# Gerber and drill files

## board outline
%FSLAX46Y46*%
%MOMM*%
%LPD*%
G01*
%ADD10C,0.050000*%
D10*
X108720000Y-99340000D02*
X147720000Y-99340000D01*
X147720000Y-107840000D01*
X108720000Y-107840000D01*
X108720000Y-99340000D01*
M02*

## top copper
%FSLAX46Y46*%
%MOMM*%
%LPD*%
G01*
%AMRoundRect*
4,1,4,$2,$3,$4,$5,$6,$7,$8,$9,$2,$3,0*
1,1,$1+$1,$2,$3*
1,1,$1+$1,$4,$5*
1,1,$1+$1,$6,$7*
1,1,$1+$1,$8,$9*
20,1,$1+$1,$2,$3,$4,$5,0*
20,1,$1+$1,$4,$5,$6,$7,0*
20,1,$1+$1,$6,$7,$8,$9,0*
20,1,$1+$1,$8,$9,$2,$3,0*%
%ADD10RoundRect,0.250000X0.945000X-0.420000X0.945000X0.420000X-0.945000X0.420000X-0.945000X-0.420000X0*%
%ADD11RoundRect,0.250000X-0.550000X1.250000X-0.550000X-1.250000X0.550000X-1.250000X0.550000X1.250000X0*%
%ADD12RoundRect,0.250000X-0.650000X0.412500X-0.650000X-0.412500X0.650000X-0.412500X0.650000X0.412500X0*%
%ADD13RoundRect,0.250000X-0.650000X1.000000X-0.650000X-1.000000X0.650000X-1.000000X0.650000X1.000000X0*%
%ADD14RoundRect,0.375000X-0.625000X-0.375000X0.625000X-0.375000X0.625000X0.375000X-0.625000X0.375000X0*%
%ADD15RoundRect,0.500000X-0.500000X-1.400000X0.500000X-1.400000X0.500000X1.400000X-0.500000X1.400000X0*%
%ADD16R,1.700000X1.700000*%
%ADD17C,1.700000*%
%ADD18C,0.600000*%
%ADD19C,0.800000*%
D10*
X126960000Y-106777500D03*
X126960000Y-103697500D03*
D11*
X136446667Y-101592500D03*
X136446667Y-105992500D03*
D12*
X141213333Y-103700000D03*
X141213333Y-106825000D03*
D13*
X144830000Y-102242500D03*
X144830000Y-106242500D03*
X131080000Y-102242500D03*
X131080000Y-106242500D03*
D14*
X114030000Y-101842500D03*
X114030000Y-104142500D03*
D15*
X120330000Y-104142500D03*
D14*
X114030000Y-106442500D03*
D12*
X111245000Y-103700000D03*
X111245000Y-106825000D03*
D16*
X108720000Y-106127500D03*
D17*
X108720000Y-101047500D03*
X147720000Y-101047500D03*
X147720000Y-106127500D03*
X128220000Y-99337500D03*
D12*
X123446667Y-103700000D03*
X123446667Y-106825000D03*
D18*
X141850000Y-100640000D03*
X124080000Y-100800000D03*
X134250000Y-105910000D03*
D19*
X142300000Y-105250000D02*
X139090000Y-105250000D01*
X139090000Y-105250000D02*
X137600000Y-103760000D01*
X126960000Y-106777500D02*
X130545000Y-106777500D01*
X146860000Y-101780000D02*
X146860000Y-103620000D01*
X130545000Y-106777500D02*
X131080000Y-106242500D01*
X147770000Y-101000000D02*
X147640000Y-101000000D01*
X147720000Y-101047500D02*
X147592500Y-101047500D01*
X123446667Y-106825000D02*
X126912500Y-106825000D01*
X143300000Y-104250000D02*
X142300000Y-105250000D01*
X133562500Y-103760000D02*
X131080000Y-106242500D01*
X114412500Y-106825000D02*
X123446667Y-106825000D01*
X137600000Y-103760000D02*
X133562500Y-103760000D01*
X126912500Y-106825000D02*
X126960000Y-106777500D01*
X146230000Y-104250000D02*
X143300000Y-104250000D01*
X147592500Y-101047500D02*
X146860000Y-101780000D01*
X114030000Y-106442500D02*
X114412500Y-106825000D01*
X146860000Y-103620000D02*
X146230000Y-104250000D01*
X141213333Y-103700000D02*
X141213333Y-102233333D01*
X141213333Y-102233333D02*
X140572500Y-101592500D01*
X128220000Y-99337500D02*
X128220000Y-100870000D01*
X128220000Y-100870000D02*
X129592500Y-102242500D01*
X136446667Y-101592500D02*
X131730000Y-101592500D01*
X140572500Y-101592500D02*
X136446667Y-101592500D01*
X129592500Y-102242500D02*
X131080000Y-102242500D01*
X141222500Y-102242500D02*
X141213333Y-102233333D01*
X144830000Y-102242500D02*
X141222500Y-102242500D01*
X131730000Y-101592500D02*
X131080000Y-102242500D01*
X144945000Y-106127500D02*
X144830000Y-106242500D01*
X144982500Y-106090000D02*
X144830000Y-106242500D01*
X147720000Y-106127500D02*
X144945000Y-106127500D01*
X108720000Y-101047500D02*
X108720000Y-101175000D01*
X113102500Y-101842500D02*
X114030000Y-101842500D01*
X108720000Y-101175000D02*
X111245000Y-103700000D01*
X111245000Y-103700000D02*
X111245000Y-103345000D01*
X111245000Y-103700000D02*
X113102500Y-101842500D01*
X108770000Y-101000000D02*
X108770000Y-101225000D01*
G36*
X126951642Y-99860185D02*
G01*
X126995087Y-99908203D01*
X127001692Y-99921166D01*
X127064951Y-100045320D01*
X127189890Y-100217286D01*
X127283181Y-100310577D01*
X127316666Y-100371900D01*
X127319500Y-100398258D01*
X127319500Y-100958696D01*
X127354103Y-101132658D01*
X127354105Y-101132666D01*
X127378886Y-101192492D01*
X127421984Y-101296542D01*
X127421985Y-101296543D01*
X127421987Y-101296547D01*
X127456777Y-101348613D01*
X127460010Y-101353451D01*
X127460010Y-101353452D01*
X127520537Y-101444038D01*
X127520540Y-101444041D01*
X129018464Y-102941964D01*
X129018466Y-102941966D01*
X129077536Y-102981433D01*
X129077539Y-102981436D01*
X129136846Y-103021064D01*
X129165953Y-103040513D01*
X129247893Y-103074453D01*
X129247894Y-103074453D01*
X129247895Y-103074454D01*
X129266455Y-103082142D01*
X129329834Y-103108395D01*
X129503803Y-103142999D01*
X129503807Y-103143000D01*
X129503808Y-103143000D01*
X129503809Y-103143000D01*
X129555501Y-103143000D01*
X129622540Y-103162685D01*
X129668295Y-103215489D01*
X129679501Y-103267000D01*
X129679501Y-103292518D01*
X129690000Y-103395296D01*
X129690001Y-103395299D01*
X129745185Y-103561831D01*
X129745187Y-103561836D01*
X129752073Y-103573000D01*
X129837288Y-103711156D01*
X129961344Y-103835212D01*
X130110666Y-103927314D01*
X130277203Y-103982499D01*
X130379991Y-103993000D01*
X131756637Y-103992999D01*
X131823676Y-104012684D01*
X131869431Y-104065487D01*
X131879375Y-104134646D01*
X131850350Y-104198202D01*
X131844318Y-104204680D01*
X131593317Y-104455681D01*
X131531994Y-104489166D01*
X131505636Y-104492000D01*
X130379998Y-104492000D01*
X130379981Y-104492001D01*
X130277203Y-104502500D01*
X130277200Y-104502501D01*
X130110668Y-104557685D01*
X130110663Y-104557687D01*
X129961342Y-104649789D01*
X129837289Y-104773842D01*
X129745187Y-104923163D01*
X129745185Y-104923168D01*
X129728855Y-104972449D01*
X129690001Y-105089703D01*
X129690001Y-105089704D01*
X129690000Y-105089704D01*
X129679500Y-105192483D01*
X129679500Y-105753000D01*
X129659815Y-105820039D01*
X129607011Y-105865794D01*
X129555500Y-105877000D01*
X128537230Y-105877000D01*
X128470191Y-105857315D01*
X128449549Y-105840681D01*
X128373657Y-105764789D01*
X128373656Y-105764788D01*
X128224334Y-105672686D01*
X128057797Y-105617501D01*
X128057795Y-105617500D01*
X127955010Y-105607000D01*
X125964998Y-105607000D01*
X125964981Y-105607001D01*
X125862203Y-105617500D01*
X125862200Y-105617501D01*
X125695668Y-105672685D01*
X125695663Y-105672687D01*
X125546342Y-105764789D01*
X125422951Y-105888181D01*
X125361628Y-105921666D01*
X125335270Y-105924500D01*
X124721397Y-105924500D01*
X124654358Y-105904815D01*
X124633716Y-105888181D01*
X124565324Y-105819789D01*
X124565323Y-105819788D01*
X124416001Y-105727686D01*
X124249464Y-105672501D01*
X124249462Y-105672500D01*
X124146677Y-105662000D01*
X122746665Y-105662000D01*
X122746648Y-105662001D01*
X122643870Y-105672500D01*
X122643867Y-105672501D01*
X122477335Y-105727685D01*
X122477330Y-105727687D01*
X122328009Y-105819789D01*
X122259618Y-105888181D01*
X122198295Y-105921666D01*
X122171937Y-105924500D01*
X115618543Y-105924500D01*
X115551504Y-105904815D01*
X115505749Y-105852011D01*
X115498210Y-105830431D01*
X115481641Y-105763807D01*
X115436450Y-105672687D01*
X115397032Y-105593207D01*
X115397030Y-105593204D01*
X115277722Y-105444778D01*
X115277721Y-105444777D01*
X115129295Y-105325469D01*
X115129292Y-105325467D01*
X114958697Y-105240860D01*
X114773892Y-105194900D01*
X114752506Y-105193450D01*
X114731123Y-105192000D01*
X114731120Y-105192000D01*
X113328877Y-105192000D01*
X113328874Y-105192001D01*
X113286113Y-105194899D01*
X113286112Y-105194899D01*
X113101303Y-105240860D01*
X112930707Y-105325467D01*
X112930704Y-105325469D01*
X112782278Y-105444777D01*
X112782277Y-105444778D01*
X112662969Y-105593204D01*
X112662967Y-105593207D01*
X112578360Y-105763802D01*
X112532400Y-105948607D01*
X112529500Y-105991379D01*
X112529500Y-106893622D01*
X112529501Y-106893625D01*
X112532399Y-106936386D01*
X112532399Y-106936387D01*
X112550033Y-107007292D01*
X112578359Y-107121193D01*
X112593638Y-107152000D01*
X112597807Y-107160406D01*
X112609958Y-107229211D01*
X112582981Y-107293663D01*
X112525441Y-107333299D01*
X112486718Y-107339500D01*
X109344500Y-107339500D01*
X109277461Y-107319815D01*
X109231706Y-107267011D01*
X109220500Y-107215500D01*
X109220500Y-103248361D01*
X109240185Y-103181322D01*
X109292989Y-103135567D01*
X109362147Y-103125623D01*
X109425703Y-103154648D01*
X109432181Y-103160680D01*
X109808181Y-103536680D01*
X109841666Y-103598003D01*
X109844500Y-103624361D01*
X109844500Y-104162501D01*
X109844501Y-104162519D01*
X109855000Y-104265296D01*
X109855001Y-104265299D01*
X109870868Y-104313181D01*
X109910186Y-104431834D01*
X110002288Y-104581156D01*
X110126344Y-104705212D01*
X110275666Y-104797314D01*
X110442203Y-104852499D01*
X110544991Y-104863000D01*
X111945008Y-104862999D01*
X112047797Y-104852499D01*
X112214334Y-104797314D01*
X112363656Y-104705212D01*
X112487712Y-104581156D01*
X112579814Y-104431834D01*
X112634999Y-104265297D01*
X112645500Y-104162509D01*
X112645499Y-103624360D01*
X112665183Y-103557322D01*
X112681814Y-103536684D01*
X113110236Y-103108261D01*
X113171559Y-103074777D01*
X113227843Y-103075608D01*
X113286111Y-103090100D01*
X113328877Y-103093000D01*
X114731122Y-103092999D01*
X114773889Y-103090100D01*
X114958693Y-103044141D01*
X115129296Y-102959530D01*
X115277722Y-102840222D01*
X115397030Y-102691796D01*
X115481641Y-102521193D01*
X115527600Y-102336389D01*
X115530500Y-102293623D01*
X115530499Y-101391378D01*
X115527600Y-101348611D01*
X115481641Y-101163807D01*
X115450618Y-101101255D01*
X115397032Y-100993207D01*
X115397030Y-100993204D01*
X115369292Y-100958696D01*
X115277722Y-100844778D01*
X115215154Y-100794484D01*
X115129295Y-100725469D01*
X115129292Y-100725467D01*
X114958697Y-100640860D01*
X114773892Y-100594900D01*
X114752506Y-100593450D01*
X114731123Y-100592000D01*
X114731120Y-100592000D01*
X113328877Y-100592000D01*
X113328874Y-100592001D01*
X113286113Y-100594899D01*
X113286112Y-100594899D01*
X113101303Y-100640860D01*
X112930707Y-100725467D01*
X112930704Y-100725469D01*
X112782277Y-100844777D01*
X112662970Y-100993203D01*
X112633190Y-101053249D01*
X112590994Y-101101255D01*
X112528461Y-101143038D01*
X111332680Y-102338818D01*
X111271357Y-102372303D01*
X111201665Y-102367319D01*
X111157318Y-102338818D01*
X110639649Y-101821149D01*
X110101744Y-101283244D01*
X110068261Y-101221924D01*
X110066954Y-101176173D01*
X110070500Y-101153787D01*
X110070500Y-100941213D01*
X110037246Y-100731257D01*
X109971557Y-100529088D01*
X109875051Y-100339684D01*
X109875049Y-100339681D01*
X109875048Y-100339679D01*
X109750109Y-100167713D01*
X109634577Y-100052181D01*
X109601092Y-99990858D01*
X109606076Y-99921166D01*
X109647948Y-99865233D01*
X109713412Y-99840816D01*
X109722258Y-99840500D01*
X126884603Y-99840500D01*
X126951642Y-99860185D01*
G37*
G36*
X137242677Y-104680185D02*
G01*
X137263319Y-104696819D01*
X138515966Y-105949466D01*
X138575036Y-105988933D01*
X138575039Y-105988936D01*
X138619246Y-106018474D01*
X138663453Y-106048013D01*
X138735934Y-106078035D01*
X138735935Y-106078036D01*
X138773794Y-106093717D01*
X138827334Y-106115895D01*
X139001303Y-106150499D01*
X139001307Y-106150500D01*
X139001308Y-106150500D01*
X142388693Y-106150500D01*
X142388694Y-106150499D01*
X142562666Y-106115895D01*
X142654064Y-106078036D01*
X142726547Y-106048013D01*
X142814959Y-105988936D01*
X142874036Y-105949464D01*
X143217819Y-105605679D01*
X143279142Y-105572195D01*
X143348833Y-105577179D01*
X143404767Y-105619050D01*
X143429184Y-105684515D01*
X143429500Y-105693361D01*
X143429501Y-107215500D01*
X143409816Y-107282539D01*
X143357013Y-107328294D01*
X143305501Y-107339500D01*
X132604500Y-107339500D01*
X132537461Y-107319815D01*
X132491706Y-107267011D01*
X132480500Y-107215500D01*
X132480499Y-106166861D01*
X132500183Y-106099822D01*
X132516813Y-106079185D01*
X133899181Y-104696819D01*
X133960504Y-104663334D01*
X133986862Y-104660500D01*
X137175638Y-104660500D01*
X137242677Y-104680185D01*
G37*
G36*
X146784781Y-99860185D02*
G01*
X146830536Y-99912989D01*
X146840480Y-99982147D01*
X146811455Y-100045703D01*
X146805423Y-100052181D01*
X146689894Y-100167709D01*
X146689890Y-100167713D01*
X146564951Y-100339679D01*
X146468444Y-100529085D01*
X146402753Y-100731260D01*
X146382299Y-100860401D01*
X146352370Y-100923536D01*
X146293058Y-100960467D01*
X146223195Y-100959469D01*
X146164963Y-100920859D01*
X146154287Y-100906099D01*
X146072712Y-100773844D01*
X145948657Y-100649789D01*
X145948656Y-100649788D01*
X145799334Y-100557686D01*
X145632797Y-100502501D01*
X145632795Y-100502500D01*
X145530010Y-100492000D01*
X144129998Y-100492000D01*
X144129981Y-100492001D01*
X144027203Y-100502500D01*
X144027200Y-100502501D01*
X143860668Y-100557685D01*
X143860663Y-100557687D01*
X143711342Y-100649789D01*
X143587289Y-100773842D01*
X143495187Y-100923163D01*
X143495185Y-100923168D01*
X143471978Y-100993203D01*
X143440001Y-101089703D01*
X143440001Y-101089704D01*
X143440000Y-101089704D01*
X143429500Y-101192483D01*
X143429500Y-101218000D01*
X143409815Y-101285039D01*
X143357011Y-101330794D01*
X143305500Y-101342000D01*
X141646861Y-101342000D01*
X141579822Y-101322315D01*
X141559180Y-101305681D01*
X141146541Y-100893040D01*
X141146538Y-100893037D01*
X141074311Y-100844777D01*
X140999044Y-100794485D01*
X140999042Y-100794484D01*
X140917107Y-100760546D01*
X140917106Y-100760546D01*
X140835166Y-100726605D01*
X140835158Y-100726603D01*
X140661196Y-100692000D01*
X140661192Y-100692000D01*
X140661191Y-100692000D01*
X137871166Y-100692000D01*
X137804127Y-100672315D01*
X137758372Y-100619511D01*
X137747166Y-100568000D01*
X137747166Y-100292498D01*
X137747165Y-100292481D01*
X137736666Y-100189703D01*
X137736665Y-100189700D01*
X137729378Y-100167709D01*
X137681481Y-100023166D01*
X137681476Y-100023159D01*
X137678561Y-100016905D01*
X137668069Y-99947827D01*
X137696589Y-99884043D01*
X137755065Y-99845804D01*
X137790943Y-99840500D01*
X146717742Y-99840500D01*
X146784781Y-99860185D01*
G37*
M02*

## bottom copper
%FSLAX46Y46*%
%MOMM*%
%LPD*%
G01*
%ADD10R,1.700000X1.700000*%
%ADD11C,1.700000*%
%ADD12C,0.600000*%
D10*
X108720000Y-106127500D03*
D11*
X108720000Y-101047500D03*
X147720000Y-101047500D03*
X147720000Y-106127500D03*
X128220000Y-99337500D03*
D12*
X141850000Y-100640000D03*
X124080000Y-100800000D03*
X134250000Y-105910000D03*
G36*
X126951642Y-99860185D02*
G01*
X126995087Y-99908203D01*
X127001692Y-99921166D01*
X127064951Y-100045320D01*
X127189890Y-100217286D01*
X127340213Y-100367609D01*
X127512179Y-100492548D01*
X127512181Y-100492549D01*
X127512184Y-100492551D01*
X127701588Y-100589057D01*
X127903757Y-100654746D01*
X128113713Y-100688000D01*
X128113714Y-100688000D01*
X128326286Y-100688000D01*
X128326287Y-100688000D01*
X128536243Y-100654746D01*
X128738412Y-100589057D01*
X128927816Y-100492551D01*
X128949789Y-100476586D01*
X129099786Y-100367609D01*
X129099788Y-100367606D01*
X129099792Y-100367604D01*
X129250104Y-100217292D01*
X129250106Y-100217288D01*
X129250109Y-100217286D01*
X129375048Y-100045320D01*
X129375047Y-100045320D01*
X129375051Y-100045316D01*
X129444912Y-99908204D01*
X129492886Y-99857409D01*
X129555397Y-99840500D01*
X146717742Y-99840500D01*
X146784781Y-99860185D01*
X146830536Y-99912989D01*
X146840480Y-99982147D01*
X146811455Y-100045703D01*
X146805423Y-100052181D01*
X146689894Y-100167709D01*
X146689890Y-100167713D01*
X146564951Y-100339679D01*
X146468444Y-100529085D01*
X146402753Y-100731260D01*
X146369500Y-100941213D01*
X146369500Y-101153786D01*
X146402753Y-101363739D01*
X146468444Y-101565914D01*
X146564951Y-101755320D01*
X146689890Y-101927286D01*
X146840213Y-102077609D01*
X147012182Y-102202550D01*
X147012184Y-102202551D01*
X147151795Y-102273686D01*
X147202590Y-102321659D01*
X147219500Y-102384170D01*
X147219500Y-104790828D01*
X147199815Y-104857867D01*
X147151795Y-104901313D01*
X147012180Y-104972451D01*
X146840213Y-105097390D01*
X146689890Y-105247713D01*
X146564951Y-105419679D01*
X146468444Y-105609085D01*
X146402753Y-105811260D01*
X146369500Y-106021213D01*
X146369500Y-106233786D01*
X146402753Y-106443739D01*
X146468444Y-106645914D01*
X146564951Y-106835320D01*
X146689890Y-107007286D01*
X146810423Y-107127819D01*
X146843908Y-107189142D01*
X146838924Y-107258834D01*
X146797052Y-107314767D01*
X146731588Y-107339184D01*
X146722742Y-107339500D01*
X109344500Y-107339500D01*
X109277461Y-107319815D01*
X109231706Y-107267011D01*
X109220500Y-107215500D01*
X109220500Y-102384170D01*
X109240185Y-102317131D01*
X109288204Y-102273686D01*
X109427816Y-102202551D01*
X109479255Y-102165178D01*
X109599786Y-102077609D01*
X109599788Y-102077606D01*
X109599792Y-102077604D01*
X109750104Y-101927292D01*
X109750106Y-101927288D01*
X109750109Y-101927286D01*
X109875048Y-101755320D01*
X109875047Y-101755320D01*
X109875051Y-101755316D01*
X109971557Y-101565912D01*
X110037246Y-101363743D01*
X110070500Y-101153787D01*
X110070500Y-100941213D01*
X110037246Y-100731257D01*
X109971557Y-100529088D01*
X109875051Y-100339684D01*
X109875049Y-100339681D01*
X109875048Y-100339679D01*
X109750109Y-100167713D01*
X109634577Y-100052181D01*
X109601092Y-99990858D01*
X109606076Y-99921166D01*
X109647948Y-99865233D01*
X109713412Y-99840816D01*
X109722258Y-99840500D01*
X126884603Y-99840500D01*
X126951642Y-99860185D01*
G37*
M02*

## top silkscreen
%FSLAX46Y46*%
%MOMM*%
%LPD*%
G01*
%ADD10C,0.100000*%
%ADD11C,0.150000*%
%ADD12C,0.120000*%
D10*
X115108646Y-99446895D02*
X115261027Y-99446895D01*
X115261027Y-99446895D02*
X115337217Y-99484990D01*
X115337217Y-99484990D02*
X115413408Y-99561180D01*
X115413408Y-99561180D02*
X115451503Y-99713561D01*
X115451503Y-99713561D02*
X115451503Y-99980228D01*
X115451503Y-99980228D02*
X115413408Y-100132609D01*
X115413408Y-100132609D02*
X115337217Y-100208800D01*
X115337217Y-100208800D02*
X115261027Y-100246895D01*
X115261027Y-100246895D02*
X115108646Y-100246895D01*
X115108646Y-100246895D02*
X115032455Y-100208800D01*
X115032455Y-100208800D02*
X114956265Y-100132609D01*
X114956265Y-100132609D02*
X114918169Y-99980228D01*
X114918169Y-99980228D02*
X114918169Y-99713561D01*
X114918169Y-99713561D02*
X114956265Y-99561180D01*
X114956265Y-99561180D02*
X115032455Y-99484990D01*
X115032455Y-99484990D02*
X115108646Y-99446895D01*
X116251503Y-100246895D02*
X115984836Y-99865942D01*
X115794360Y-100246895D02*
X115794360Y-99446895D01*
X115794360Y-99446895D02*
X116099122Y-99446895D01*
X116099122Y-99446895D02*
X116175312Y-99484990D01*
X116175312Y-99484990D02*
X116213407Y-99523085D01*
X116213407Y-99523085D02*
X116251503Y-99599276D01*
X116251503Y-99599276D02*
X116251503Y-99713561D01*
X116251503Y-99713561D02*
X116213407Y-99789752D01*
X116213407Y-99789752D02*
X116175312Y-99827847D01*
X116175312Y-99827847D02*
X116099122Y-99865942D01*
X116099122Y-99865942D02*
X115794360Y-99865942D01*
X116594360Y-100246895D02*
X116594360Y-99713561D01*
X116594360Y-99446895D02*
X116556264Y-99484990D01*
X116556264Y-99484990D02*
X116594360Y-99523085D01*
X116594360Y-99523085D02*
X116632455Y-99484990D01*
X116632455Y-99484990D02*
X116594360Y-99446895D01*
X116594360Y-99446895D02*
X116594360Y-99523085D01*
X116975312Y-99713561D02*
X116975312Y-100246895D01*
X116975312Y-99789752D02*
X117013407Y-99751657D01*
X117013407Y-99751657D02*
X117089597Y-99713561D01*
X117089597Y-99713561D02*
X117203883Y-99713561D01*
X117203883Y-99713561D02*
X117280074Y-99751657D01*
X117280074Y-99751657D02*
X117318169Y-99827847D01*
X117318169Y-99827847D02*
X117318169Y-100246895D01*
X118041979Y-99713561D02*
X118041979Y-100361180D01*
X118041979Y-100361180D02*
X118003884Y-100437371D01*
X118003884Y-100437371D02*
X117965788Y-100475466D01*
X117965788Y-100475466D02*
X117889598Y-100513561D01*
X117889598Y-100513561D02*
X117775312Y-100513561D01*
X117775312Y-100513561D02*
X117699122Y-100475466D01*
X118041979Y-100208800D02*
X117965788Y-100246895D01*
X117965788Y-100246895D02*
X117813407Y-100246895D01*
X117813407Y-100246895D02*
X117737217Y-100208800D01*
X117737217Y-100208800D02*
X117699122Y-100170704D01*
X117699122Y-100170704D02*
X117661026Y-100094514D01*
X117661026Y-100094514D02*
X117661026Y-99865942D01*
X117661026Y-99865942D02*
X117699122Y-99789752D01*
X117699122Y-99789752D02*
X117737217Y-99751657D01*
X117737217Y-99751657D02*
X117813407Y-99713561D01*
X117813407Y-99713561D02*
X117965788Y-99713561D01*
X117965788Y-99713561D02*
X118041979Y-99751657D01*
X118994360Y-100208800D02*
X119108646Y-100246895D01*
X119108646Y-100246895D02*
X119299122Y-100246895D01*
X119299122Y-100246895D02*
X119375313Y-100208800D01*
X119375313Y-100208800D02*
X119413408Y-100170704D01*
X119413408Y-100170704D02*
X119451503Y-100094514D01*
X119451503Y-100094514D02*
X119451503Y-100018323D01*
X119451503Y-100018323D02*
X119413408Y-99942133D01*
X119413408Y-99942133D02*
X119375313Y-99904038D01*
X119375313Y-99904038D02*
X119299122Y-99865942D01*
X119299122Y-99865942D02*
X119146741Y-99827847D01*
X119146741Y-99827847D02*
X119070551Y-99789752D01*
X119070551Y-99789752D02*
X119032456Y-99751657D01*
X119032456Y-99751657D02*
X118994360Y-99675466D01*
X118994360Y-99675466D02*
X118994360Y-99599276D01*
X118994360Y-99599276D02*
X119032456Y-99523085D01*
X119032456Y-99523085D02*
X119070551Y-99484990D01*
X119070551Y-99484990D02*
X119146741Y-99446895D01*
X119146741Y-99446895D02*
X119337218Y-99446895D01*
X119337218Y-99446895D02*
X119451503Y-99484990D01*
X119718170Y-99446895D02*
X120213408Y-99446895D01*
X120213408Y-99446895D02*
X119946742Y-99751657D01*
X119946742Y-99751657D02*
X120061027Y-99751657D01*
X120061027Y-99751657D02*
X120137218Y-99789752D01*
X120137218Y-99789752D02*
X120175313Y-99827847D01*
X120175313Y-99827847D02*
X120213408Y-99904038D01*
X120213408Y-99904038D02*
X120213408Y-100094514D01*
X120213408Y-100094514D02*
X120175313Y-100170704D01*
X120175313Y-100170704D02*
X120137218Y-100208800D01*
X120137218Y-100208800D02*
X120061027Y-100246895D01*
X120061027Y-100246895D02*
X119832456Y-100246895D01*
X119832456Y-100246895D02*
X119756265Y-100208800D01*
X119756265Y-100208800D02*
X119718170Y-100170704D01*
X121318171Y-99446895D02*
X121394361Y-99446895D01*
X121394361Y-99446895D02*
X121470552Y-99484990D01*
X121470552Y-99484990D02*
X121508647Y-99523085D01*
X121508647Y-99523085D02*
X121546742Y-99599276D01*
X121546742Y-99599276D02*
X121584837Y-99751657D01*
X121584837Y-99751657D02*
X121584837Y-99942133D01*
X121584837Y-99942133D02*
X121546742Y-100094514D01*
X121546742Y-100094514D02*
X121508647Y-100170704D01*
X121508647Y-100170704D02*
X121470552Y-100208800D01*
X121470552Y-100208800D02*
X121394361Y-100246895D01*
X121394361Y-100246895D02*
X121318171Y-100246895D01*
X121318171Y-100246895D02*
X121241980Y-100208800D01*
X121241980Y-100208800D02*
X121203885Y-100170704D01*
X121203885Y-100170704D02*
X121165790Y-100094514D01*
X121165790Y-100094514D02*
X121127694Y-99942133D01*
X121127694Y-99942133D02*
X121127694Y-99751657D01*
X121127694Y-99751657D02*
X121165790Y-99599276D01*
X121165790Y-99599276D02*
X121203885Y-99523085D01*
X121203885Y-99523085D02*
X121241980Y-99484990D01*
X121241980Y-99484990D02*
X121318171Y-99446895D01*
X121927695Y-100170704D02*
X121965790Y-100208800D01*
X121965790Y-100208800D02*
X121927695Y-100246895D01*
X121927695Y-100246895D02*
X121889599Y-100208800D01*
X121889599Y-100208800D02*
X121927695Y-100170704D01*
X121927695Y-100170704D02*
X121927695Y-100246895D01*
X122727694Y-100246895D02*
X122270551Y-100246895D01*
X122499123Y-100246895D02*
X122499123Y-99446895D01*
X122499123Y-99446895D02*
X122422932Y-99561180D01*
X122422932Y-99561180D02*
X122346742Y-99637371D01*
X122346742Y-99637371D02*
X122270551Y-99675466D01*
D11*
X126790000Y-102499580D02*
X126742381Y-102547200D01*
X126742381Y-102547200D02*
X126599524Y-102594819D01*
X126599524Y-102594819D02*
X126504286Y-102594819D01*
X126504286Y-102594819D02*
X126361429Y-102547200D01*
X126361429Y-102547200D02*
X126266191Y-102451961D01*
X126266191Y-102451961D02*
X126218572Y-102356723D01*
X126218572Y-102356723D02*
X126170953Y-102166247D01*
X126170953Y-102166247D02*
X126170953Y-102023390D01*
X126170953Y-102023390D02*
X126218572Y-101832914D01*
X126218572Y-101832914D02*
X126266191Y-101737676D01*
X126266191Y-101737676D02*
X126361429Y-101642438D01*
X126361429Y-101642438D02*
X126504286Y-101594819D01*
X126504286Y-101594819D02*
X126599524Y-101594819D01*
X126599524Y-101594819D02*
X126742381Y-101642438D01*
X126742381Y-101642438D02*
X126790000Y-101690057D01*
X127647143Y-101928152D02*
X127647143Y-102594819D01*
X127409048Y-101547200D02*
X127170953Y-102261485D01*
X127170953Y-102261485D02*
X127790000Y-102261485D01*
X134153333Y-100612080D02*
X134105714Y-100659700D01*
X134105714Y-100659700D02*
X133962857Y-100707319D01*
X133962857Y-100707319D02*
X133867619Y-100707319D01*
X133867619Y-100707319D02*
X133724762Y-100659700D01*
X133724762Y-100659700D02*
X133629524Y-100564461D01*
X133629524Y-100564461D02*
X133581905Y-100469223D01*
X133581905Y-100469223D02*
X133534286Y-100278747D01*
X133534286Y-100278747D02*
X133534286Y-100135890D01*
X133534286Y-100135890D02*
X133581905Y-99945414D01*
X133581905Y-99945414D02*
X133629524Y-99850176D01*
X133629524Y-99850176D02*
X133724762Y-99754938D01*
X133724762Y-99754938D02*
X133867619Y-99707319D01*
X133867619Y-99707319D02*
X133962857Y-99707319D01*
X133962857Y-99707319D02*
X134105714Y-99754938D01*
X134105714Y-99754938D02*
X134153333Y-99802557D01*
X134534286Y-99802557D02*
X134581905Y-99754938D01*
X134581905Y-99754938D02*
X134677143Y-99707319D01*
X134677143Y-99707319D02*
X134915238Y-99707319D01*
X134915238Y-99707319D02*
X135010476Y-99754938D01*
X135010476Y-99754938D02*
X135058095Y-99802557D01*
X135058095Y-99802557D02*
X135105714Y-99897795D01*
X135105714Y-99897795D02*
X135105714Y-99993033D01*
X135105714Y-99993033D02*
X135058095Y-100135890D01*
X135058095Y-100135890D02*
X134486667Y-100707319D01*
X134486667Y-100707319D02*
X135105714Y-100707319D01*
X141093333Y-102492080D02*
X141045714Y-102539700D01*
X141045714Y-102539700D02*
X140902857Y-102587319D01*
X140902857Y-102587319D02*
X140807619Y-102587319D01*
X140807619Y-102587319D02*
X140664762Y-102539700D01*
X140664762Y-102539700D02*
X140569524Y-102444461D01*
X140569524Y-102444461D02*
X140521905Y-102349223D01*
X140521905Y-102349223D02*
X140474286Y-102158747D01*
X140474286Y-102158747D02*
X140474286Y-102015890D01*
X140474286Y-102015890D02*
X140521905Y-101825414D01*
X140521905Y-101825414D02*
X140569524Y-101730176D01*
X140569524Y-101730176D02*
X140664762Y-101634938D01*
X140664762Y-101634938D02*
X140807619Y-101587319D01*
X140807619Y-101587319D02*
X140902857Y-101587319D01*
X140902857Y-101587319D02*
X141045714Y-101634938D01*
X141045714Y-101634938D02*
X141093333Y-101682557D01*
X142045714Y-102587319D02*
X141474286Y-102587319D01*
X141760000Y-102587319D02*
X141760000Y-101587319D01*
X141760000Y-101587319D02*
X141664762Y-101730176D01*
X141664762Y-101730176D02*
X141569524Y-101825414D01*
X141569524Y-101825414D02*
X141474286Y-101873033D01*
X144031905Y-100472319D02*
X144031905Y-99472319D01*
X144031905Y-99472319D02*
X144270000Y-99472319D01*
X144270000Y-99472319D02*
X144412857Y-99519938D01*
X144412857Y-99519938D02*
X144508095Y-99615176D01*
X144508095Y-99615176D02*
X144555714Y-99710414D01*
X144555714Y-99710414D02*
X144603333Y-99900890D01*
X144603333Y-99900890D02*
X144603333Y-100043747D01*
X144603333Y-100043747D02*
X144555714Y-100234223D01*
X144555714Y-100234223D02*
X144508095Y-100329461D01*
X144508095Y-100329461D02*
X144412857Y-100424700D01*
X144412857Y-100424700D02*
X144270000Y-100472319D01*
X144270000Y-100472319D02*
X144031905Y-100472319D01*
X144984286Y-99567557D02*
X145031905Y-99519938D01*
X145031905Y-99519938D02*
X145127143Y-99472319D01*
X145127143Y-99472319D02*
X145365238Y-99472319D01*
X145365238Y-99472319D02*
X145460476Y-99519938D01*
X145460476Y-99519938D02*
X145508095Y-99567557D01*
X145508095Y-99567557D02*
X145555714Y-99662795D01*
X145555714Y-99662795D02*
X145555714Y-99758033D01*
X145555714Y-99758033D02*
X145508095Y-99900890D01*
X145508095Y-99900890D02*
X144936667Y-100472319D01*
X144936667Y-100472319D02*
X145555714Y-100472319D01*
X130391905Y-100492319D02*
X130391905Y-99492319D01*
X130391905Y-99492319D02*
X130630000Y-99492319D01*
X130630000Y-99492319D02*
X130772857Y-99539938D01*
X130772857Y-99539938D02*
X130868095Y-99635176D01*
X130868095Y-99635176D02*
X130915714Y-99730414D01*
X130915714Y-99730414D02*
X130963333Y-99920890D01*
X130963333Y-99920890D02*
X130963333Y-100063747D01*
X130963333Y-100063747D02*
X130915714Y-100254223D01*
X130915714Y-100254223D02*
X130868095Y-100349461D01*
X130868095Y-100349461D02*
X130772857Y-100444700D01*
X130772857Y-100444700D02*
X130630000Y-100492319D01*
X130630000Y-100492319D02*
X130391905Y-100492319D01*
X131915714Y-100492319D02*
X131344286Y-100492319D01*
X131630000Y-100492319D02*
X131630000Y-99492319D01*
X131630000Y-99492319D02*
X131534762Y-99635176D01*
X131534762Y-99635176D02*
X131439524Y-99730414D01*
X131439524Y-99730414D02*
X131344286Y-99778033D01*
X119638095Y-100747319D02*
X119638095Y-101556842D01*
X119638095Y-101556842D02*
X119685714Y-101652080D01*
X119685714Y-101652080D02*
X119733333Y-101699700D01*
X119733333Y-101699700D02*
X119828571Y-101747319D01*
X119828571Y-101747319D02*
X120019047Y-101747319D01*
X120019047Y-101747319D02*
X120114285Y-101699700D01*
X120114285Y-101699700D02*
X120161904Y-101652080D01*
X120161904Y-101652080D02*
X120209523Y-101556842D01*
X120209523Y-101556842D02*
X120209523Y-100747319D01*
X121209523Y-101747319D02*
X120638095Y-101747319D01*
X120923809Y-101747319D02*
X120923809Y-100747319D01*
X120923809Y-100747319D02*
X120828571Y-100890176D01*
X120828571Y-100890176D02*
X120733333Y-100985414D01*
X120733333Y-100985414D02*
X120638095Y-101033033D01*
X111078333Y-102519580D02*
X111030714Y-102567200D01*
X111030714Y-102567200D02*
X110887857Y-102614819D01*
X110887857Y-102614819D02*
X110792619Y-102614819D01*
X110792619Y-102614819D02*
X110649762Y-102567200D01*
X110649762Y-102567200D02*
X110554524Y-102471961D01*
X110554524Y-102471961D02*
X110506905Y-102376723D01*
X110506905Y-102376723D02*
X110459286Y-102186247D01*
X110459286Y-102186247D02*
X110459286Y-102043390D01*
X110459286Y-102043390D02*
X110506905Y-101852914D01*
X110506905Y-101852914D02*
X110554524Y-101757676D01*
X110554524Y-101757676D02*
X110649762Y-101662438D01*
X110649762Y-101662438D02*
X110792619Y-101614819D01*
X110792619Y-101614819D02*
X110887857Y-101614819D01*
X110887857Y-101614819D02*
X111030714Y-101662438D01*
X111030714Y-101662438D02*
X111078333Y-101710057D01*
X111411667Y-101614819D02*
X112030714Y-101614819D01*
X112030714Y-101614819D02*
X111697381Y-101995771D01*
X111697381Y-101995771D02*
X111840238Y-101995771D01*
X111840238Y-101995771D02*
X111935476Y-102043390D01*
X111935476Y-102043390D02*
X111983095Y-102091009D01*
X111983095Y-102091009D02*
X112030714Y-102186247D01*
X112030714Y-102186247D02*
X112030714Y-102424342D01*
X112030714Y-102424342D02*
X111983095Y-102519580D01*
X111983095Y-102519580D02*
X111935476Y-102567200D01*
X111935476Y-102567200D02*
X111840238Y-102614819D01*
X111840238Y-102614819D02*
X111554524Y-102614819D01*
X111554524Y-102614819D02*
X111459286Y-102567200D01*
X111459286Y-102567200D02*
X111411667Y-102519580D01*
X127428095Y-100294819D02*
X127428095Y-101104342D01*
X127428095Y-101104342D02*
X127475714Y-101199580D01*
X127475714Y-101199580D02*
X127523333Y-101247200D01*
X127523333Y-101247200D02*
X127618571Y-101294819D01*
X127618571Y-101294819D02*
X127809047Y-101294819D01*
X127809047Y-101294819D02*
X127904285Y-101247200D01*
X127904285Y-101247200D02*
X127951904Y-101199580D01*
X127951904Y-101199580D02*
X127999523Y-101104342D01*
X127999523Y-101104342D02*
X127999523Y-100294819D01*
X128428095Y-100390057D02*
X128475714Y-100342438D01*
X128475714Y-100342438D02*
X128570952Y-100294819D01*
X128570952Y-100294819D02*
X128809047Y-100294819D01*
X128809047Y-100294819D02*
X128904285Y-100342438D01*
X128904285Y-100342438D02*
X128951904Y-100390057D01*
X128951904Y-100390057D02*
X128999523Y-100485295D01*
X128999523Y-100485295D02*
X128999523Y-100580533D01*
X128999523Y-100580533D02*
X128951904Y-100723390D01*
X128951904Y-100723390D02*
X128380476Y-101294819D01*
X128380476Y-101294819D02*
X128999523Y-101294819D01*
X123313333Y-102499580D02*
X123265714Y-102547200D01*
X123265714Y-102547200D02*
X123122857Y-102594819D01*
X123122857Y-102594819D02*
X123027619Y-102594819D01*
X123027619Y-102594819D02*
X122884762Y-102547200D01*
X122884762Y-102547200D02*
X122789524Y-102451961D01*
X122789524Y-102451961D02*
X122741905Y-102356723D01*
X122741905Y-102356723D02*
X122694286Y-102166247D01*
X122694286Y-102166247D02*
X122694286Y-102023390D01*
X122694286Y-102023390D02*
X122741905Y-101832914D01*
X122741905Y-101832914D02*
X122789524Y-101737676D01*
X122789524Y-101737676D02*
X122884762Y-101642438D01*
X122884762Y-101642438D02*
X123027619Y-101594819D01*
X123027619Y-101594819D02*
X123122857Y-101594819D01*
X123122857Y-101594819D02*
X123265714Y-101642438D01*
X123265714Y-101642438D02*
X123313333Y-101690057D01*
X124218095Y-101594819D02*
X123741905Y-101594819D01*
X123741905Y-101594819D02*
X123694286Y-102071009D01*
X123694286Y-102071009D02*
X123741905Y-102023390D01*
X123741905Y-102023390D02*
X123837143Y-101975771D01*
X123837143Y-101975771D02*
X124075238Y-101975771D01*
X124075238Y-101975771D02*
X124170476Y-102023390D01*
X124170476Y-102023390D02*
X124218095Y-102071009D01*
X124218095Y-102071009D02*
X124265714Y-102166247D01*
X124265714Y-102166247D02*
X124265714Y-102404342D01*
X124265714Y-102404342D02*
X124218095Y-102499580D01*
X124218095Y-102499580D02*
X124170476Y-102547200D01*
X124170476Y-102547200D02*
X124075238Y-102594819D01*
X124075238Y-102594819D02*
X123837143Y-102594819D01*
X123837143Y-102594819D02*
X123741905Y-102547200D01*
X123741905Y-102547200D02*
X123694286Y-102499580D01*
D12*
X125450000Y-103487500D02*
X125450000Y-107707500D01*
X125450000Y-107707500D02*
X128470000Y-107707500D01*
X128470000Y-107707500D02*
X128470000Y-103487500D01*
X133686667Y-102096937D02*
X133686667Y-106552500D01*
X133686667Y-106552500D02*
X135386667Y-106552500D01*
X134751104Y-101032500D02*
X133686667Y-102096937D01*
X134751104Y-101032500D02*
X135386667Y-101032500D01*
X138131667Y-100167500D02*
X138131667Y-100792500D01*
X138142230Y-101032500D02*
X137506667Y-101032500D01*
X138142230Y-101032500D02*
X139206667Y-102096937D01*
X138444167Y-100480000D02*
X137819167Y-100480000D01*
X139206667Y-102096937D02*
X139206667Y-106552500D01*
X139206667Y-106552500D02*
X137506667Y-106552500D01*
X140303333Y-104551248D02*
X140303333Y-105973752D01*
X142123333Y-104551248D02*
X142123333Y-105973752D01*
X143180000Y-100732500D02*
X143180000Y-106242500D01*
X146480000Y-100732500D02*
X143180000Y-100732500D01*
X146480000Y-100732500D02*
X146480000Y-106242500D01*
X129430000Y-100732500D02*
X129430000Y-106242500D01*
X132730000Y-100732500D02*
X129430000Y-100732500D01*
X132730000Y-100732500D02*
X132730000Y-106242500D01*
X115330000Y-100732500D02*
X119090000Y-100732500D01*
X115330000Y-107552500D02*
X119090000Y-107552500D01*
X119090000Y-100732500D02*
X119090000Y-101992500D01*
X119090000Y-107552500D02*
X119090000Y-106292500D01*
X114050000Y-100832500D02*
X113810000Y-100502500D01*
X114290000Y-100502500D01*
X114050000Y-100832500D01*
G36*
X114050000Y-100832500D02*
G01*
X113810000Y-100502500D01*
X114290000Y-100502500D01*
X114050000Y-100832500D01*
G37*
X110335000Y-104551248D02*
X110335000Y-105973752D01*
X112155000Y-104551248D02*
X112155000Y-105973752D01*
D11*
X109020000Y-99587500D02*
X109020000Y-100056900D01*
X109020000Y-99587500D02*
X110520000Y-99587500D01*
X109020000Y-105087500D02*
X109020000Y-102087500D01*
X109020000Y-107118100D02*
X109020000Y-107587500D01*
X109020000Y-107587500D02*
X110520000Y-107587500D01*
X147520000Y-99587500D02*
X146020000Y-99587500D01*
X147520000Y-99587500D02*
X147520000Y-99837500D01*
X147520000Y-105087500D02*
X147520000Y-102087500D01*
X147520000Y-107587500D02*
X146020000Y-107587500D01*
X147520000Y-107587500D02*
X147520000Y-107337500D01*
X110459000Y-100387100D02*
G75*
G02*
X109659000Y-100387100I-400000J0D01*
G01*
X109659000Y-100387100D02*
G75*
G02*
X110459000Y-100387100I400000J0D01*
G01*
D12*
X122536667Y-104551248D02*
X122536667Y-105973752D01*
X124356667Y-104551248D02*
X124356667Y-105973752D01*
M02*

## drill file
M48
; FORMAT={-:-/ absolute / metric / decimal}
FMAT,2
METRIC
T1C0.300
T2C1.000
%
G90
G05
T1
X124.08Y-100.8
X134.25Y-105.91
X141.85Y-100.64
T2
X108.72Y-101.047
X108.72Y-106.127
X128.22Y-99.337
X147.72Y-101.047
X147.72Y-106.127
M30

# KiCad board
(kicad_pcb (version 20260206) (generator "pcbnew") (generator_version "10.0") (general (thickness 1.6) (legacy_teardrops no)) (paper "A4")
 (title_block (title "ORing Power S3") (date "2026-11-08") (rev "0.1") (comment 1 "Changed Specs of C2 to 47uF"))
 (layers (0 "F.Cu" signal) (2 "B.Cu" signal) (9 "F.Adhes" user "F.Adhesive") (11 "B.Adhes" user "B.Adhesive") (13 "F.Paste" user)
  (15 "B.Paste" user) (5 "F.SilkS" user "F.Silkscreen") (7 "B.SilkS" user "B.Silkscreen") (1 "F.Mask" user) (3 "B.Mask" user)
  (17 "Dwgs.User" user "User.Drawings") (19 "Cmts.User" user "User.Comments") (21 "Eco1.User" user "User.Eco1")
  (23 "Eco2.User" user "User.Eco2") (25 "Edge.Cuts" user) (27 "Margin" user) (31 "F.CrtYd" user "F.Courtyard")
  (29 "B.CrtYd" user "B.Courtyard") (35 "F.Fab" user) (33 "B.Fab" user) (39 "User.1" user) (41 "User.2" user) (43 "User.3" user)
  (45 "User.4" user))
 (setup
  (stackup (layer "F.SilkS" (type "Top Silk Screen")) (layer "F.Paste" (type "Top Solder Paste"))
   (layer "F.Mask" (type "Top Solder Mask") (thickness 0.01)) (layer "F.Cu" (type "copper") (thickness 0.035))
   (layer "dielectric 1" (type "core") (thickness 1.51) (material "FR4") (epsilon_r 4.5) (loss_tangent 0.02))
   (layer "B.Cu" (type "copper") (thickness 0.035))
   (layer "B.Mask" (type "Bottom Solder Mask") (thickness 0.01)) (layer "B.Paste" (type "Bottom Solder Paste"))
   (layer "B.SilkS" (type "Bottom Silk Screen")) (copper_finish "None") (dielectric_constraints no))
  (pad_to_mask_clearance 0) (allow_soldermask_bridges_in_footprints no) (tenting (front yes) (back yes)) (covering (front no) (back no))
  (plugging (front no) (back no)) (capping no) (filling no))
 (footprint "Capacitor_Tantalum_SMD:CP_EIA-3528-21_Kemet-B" (layer "F.Cu") (at 126.96 105.2375 90)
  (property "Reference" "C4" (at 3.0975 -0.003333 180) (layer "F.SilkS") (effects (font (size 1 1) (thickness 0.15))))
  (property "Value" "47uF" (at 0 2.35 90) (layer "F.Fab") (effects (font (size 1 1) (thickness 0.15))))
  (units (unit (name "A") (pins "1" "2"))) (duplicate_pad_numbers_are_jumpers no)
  (fp_line (start 1.75 -1.51) (end -2.47 -1.51) (stroke (width 0.12) (type solid)) (layer "F.SilkS"))
  (fp_line (start -2.47 -1.51) (end -2.47 1.51) (stroke (width 0.12) (type solid)) (layer "F.SilkS"))
  (fp_line (start -2.47 1.51) (end 1.75 1.51) (stroke (width 0.12) (type solid)) (layer "F.SilkS"))
  (pad "1" smd roundrect (at -1.54 0 90) (size 1.34 2.39) (layers "F.Cu" "F.Mask" "F.Paste") (roundrect_rratio 0.186567) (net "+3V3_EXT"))
  (pad "2" smd roundrect (at 1.54 0 90) (size 1.34 2.39) (layers "F.Cu" "F.Mask" "F.Paste") (roundrect_rratio 0.186567) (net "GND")
   (zone_connect 2)))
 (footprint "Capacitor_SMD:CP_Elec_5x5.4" (layer "F.Cu") (at 136.446667 103.7925 -90)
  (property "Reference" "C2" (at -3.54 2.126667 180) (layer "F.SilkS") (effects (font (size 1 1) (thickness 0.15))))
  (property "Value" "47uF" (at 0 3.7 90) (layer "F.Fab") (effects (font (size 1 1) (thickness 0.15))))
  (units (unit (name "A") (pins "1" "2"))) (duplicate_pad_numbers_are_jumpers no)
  (fp_line (start -1.695563 2.76) (end 2.76 2.76) (stroke (width 0.12) (type solid)) (layer "F.SilkS"))
  (fp_line (start 2.76 2.76) (end 2.76 1.06) (stroke (width 0.12) (type solid)) (layer "F.SilkS"))
  (fp_line (start -2.76 1.695563) (end -1.695563 2.76) (stroke (width 0.12) (type solid)) (layer "F.SilkS"))
  (fp_line (start -2.76 1.695563) (end -2.76 1.06) (stroke (width 0.12) (type solid)) (layer "F.SilkS"))
  (fp_line (start -3.625 -1.685) (end -3 -1.685) (stroke (width 0.12) (type solid)) (layer "F.SilkS"))
  (fp_line (start -2.76 -1.695563) (end -2.76 -1.06) (stroke (width 0.12) (type solid)) (layer "F.SilkS"))
  (fp_line (start -2.76 -1.695563) (end -1.695563 -2.76) (stroke (width 0.12) (type solid)) (layer "F.SilkS"))
  (fp_line (start -3.3125 -1.9975) (end -3.3125 -1.3725) (stroke (width 0.12) (type solid)) (layer "F.SilkS"))
  (fp_line (start -1.695563 -2.76) (end 2.76 -2.76) (stroke (width 0.12) (type solid)) (layer "F.SilkS"))
  (fp_line (start 2.76 -2.76) (end 2.76 -1.06) (stroke (width 0.12) (type solid)) (layer "F.SilkS"))
  (pad "1" smd roundrect (at -2.2 0 270) (size 3 1.6) (layers "F.Cu" "F.Mask" "F.Paste") (roundrect_rratio 0.15625) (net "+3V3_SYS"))
  (pad "2" smd roundrect (at 2.2 0 270) (size 3 1.6) (layers "F.Cu" "F.Mask" "F.Paste") (roundrect_rratio 0.15625) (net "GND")
   (zone_connect 2)))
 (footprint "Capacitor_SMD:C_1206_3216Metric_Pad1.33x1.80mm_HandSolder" (layer "F.Cu") (at 141.213333 105.2625 -90)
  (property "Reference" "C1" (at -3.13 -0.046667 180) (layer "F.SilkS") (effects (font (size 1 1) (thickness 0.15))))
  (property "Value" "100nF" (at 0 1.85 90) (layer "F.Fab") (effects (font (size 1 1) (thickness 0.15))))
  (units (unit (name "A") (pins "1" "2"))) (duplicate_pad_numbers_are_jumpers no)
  (fp_line (start -0.711252 0.91) (end 0.711252 0.91) (stroke (width 0.12) (type solid)) (layer "F.SilkS"))
  (fp_line (start -0.711252 -0.91) (end 0.711252 -0.91) (stroke (width 0.12) (type solid)) (layer "F.SilkS"))
  (pad "1" smd roundrect (at -1.5625 0 270) (size 1.325 1.8) (layers "F.Cu" "F.Mask" "F.Paste") (roundrect_rratio 0.188679) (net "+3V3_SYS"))
  (pad "2" smd roundrect (at 1.5625 0 270) (size 1.325 1.8) (layers "F.Cu" "F.Mask" "F.Paste") (roundrect_rratio 0.188679) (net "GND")
   (zone_connect 2)))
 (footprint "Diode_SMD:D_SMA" (layer "F.Cu") (at 144.83 104.2425 -90)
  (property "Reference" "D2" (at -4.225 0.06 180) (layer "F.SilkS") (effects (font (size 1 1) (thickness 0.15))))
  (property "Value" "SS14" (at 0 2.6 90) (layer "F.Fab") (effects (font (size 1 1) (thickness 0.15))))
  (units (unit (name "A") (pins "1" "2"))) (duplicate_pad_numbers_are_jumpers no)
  (fp_line (start -3.51 1.65) (end 2 1.65) (stroke (width 0.12) (type solid)) (layer "F.SilkS"))
  (fp_line (start -3.51 -1.65) (end -3.51 1.65) (stroke (width 0.12) (type solid)) (layer "F.SilkS"))
  (fp_line (start -3.51 -1.65) (end 2 -1.65) (stroke (width 0.12) (type solid)) (layer "F.SilkS"))
  (pad "1" smd roundrect (at -2 0 270) (size 2.5 1.8) (layers "F.Cu" "F.Mask" "F.Paste") (roundrect_rratio 0.1388888889) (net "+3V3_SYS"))
  (pad "2" smd roundrect (at 2 0 270) (size 2.5 1.8) (layers "F.Cu" "F.Mask" "F.Paste") (roundrect_rratio 0.1388888889) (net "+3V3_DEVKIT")))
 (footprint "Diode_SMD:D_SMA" (layer "F.Cu") (at 131.08 104.2425 -90)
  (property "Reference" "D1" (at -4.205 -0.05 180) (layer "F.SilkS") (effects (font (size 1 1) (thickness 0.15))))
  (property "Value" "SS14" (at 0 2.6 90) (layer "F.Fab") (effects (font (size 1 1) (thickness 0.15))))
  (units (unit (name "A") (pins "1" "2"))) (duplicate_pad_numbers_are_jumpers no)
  (fp_line (start -3.51 1.65) (end 2 1.65) (stroke (width 0.12) (type solid)) (layer "F.SilkS"))
  (fp_line (start -3.51 -1.65) (end -3.51 1.65) (stroke (width 0.12) (type solid)) (layer "F.SilkS"))
  (fp_line (start -3.51 -1.65) (end 2 -1.65) (stroke (width 0.12) (type solid)) (layer "F.SilkS"))
  (pad "1" smd roundrect (at -2 0 270) (size 2.5 1.8) (layers "F.Cu" "F.Mask" "F.Paste") (roundrect_rratio 0.1388888889) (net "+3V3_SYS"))
  (pad "2" smd roundrect (at 2 0 270) (size 2.5 1.8) (layers "F.Cu" "F.Mask" "F.Paste") (roundrect_rratio 0.1388888889) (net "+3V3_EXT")))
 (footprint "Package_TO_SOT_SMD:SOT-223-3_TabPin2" (layer "F.Cu") (at 117.18 104.1425)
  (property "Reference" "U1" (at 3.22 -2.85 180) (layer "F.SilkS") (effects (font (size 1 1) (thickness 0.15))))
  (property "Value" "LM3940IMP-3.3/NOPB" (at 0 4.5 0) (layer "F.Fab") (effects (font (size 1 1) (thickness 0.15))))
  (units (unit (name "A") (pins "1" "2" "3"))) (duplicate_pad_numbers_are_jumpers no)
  (fp_line (start -1.85 -3.41) (end 1.91 -3.41) (stroke (width 0.12) (type solid)) (layer "F.SilkS"))
  (fp_line (start -1.85 3.41) (end 1.91 3.41) (stroke (width 0.12) (type solid)) (layer "F.SilkS"))
  (fp_line (start 1.91 -3.41) (end 1.91 -2.15) (stroke (width 0.12) (type solid)) (layer "F.SilkS"))
  (fp_line (start 1.91 3.41) (end 1.91 2.15) (stroke (width 0.12) (type solid)) (layer "F.SilkS"))
  (fp_poly
   (pts (xy -3.13 -3.31) (xy -3.37 -3.64) (xy -2.89 -3.64) (xy -3.13 -3.31)) (stroke (width 0.12) (type solid)) (fill yes) (layer "F.SilkS"))
  (pad "1" smd roundrect (at -3.15 -2.3) (size 2 1.5) (layers "F.Cu" "F.Mask" "F.Paste") (roundrect_rratio 0.25) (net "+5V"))
  (pad "2" smd roundrect (at -3.15 0) (size 2 1.5) (layers "F.Cu" "F.Mask" "F.Paste") (roundrect_rratio 0.25) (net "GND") (zone_connect 2))
  (pad "2" smd roundrect (at 3.15 0) (size 2 3.8) (layers "F.Cu" "F.Mask" "F.Paste") (roundrect_rratio 0.25) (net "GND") (zone_connect 2))
  (pad "3" smd roundrect (at -3.15 2.3) (size 2 1.5) (layers "F.Cu" "F.Mask" "F.Paste") (roundrect_rratio 0.25) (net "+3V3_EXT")))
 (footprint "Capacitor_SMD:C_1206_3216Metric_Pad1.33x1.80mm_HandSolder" (layer "F.Cu") (at 111.245 105.2625 -90)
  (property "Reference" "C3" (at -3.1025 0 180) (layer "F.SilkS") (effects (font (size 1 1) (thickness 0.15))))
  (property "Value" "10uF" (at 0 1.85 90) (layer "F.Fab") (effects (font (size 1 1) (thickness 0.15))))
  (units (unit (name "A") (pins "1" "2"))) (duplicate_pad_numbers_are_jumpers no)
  (fp_line (start -0.711252 0.91) (end 0.711252 0.91) (stroke (width 0.12) (type solid)) (layer "F.SilkS"))
  (fp_line (start -0.711252 -0.91) (end 0.711252 -0.91) (stroke (width 0.12) (type solid)) (layer "F.SilkS"))
  (pad "1" smd roundrect (at -1.5625 0 270) (size 1.325 1.8) (layers "F.Cu" "F.Mask" "F.Paste") (roundrect_rratio 0.188679) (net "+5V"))
  (pad "2" smd roundrect (at 1.5625 0 270) (size 1.325 1.8) (layers "F.Cu" "F.Mask" "F.Paste") (roundrect_rratio 0.188679) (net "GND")
   (zone_connect 2)))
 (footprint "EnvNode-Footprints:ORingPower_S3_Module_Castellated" (layer "F.Cu") (at 128.22 103.5875)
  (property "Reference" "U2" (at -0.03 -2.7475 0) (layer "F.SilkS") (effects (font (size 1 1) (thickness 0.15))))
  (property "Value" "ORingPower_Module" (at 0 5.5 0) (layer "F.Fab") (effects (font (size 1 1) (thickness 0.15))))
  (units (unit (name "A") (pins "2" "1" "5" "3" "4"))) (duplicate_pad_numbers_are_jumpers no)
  (fp_line (start -19.2 -4) (end -19.2 -3.5306) (stroke (width 0.15) (type solid)) (layer "F.SilkS"))
  (fp_line (start -19.2 -4) (end -17.7 -4) (stroke (width 0.15) (type solid)) (layer "F.SilkS"))
  (fp_line (start -19.2 1.5) (end -19.2 -1.5) (stroke (width 0.15) (type solid)) (layer "F.SilkS"))
  (fp_line (start -19.2 3.5306) (end -19.2 4) (stroke (width 0.15) (type solid)) (layer "F.SilkS"))
  (fp_line (start -19.2 4) (end -17.7 4) (stroke (width 0.15) (type solid)) (layer "F.SilkS"))
  (fp_line (start 19.3 -4) (end 17.8 -4) (stroke (width 0.15) (type solid)) (layer "F.SilkS"))
  (fp_line (start 19.3 -4) (end 19.3 -3.75) (stroke (width 0.15) (type solid)) (layer "F.SilkS"))
  (fp_line (start 19.3 1.5) (end 19.3 -1.5) (stroke (width 0.15) (type solid)) (layer "F.SilkS"))
  (fp_line (start 19.3 4) (end 17.8 4) (stroke (width 0.15) (type solid)) (layer "F.SilkS"))
  (fp_line (start 19.3 4) (end 19.3 3.75) (stroke (width 0.15) (type solid)) (layer "F.SilkS"))
  (fp_circle (center -18.161 -3.2004) (end -17.761 -3.2004) (stroke (width 0.15) (type solid)) (fill no) (layer "F.SilkS"))
  (pad "1" thru_hole rect (at -19.5 2.54) (size 1.7 1.7) (drill 1) (layers "*.Cu" "*.Mask") (remove_unused_layers no) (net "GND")
   (zone_connect 2))
  (pad "2" thru_hole circle (at -19.5 -2.54) (size 1.7 1.7) (drill 1) (layers "*.Cu" "*.Mask") (remove_unused_layers no) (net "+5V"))
  (pad "3" thru_hole circle (at 19.5 -2.54) (size 1.7 1.7) (drill 1) (layers "*.Cu" "*.Mask") (remove_unused_layers no) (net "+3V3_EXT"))
  (pad "4" thru_hole circle (at 19.5 2.54) (size 1.7 1.7) (drill 1) (layers "*.Cu" "*.Mask") (remove_unused_layers no) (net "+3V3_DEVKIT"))
  (pad "5" thru_hole circle (at 0 -4.25) (size 1.7 1.7) (drill 1) (layers "*.Cu" "*.Mask") (remove_unused_layers no) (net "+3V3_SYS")))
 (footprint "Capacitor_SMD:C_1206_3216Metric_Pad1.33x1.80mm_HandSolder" (layer "F.Cu") (at 123.446667 105.2625 -90)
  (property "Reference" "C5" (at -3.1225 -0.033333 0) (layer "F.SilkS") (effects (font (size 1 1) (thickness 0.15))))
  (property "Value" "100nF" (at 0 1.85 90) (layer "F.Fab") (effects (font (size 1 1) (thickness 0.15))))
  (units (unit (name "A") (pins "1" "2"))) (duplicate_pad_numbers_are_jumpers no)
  (fp_line (start -0.711252 0.91) (end 0.711252 0.91) (stroke (width 0.12) (type solid)) (layer "F.SilkS"))
  (fp_line (start -0.711252 -0.91) (end 0.711252 -0.91) (stroke (width 0.12) (type solid)) (layer "F.SilkS"))
  (pad "1" smd roundrect (at -1.5625 0 270) (size 1.325 1.8) (layers "F.Cu" "F.Mask" "F.Paste") (roundrect_rratio 0.188679) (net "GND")
   (zone_connect 2))
  (pad "2" smd roundrect (at 1.5625 0 270) (size 1.325 1.8) (layers "F.Cu" "F.Mask" "F.Paste") (roundrect_rratio 0.188679) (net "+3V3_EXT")))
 (gr_rect (start 108.72 99.34) (end 147.72 107.84) (stroke (width 0.05) (type default)) (fill no) (layer "Edge.Cuts"))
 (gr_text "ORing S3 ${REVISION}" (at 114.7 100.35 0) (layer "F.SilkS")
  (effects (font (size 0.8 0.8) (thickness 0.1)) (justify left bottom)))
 (segment (start 142.3 105.25) (end 139.09 105.25) (width 0.8) (layer "F.Cu") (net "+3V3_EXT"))
 (segment (start 139.09 105.25) (end 137.6 103.76) (width 0.8) (layer "F.Cu") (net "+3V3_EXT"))
 (segment (start 126.96 106.7775) (end 130.545 106.7775) (width 0.8) (layer "F.Cu") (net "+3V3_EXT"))
 (segment (start 146.86 101.78) (end 146.86 103.62) (width 0.8) (layer "F.Cu") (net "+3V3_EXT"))
 (segment (start 130.545 106.7775) (end 131.08 106.2425) (width 0.8) (layer "F.Cu") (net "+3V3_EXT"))
 (segment (start 147.77 101) (end 147.64 101) (width 0.8) (layer "F.Cu") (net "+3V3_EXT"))
 (segment (start 147.72 101.0475) (end 147.5925 101.0475) (width 0.8) (layer "F.Cu") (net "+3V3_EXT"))
 (segment (start 123.446667 106.825) (end 126.9125 106.825) (width 0.8) (layer "F.Cu") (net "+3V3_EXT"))
 (segment (start 143.3 104.25) (end 142.3 105.25) (width 0.8) (layer "F.Cu") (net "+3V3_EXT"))
 (segment (start 133.5625 103.76) (end 131.08 106.2425) (width 0.8) (layer "F.Cu") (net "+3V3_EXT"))
 (segment (start 114.4125 106.825) (end 123.446667 106.825) (width 0.8) (layer "F.Cu") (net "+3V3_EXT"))
 (segment (start 137.6 103.76) (end 133.5625 103.76) (width 0.8) (layer "F.Cu") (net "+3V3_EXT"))
 (segment (start 126.9125 106.825) (end 126.96 106.7775) (width 0.8) (layer "F.Cu") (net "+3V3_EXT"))
 (segment (start 146.23 104.25) (end 143.3 104.25) (width 0.8) (layer "F.Cu") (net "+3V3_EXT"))
 (segment (start 147.5925 101.0475) (end 146.86 101.78) (width 0.8) (layer "F.Cu") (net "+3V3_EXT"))
 (segment (start 114.03 106.4425) (end 114.4125 106.825) (width 0.8) (layer "F.Cu") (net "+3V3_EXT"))
 (segment (start 146.86 103.62) (end 146.23 104.25) (width 0.8) (layer "F.Cu") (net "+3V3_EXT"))
 (via (at 141.85 100.64) (size 0.6) (drill 0.3) (layers "F.Cu" "B.Cu") (free yes) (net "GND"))
 (via (at 124.08 100.8) (size 0.6) (drill 0.3) (layers "F.Cu" "B.Cu") (free yes) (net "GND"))
 (via (at 134.25 105.91) (size 0.6) (drill 0.3) (layers "F.Cu" "B.Cu") (free yes) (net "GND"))
 (segment (start 141.213333 103.7) (end 141.213333 102.233333) (width 0.8) (layer "F.Cu") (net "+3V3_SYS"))
 (segment (start 141.213333 102.233333) (end 140.5725 101.5925) (width 0.8) (layer "F.Cu") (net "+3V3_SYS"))
 (segment (start 128.22 99.3375) (end 128.22 100.87) (width 0.8) (layer "F.Cu") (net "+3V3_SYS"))
 (segment (start 128.22 100.87) (end 129.5925 102.2425) (width 0.8) (layer "F.Cu") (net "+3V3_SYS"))
 (segment (start 136.446667 101.5925) (end 131.73 101.5925) (width 0.8) (layer "F.Cu") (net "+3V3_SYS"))
 (segment (start 140.5725 101.5925) (end 136.446667 101.5925) (width 0.8) (layer "F.Cu") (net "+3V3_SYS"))
 (segment (start 129.5925 102.2425) (end 131.08 102.2425) (width 0.8) (layer "F.Cu") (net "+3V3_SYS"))
 (segment (start 141.2225 102.2425) (end 141.213333 102.233333) (width 0.8) (layer "F.Cu") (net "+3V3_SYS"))
 (segment (start 144.83 102.2425) (end 141.2225 102.2425) (width 0.8) (layer "F.Cu") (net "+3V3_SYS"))
 (segment (start 131.73 101.5925) (end 131.08 102.2425) (width 0.8) (layer "F.Cu") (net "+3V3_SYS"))
 (segment (start 144.945 106.1275) (end 144.83 106.2425) (width 0.8) (layer "F.Cu") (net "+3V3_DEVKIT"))
 (segment (start 144.9825 106.09) (end 144.83 106.2425) (width 0.8) (layer "F.Cu") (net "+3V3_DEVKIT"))
 (segment (start 147.72 106.1275) (end 144.945 106.1275) (width 0.8) (layer "F.Cu") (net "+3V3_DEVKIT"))
 (segment (start 108.72 101.0475) (end 108.72 101.175) (width 0.8) (layer "F.Cu") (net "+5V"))
 (segment (start 113.1025 101.8425) (end 114.03 101.8425) (width 0.8) (layer "F.Cu") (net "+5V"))
 (segment (start 108.72 101.175) (end 111.245 103.7) (width 0.8) (layer "F.Cu") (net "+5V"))
 (segment (start 111.245 103.7) (end 111.245 103.345) (width 0.8) (layer "F.Cu") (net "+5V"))
 (segment (start 111.245 103.7) (end 113.1025 101.8425) (width 0.8) (layer "F.Cu") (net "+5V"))
 (segment (start 108.77 101) (end 108.77 101.225) (width 0.8) (layer "F.Cu") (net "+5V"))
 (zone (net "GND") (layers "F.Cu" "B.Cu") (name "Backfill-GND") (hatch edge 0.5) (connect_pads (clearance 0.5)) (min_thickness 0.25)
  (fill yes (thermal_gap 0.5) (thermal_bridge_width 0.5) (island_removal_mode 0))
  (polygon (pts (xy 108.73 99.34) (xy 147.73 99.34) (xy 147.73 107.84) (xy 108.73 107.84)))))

